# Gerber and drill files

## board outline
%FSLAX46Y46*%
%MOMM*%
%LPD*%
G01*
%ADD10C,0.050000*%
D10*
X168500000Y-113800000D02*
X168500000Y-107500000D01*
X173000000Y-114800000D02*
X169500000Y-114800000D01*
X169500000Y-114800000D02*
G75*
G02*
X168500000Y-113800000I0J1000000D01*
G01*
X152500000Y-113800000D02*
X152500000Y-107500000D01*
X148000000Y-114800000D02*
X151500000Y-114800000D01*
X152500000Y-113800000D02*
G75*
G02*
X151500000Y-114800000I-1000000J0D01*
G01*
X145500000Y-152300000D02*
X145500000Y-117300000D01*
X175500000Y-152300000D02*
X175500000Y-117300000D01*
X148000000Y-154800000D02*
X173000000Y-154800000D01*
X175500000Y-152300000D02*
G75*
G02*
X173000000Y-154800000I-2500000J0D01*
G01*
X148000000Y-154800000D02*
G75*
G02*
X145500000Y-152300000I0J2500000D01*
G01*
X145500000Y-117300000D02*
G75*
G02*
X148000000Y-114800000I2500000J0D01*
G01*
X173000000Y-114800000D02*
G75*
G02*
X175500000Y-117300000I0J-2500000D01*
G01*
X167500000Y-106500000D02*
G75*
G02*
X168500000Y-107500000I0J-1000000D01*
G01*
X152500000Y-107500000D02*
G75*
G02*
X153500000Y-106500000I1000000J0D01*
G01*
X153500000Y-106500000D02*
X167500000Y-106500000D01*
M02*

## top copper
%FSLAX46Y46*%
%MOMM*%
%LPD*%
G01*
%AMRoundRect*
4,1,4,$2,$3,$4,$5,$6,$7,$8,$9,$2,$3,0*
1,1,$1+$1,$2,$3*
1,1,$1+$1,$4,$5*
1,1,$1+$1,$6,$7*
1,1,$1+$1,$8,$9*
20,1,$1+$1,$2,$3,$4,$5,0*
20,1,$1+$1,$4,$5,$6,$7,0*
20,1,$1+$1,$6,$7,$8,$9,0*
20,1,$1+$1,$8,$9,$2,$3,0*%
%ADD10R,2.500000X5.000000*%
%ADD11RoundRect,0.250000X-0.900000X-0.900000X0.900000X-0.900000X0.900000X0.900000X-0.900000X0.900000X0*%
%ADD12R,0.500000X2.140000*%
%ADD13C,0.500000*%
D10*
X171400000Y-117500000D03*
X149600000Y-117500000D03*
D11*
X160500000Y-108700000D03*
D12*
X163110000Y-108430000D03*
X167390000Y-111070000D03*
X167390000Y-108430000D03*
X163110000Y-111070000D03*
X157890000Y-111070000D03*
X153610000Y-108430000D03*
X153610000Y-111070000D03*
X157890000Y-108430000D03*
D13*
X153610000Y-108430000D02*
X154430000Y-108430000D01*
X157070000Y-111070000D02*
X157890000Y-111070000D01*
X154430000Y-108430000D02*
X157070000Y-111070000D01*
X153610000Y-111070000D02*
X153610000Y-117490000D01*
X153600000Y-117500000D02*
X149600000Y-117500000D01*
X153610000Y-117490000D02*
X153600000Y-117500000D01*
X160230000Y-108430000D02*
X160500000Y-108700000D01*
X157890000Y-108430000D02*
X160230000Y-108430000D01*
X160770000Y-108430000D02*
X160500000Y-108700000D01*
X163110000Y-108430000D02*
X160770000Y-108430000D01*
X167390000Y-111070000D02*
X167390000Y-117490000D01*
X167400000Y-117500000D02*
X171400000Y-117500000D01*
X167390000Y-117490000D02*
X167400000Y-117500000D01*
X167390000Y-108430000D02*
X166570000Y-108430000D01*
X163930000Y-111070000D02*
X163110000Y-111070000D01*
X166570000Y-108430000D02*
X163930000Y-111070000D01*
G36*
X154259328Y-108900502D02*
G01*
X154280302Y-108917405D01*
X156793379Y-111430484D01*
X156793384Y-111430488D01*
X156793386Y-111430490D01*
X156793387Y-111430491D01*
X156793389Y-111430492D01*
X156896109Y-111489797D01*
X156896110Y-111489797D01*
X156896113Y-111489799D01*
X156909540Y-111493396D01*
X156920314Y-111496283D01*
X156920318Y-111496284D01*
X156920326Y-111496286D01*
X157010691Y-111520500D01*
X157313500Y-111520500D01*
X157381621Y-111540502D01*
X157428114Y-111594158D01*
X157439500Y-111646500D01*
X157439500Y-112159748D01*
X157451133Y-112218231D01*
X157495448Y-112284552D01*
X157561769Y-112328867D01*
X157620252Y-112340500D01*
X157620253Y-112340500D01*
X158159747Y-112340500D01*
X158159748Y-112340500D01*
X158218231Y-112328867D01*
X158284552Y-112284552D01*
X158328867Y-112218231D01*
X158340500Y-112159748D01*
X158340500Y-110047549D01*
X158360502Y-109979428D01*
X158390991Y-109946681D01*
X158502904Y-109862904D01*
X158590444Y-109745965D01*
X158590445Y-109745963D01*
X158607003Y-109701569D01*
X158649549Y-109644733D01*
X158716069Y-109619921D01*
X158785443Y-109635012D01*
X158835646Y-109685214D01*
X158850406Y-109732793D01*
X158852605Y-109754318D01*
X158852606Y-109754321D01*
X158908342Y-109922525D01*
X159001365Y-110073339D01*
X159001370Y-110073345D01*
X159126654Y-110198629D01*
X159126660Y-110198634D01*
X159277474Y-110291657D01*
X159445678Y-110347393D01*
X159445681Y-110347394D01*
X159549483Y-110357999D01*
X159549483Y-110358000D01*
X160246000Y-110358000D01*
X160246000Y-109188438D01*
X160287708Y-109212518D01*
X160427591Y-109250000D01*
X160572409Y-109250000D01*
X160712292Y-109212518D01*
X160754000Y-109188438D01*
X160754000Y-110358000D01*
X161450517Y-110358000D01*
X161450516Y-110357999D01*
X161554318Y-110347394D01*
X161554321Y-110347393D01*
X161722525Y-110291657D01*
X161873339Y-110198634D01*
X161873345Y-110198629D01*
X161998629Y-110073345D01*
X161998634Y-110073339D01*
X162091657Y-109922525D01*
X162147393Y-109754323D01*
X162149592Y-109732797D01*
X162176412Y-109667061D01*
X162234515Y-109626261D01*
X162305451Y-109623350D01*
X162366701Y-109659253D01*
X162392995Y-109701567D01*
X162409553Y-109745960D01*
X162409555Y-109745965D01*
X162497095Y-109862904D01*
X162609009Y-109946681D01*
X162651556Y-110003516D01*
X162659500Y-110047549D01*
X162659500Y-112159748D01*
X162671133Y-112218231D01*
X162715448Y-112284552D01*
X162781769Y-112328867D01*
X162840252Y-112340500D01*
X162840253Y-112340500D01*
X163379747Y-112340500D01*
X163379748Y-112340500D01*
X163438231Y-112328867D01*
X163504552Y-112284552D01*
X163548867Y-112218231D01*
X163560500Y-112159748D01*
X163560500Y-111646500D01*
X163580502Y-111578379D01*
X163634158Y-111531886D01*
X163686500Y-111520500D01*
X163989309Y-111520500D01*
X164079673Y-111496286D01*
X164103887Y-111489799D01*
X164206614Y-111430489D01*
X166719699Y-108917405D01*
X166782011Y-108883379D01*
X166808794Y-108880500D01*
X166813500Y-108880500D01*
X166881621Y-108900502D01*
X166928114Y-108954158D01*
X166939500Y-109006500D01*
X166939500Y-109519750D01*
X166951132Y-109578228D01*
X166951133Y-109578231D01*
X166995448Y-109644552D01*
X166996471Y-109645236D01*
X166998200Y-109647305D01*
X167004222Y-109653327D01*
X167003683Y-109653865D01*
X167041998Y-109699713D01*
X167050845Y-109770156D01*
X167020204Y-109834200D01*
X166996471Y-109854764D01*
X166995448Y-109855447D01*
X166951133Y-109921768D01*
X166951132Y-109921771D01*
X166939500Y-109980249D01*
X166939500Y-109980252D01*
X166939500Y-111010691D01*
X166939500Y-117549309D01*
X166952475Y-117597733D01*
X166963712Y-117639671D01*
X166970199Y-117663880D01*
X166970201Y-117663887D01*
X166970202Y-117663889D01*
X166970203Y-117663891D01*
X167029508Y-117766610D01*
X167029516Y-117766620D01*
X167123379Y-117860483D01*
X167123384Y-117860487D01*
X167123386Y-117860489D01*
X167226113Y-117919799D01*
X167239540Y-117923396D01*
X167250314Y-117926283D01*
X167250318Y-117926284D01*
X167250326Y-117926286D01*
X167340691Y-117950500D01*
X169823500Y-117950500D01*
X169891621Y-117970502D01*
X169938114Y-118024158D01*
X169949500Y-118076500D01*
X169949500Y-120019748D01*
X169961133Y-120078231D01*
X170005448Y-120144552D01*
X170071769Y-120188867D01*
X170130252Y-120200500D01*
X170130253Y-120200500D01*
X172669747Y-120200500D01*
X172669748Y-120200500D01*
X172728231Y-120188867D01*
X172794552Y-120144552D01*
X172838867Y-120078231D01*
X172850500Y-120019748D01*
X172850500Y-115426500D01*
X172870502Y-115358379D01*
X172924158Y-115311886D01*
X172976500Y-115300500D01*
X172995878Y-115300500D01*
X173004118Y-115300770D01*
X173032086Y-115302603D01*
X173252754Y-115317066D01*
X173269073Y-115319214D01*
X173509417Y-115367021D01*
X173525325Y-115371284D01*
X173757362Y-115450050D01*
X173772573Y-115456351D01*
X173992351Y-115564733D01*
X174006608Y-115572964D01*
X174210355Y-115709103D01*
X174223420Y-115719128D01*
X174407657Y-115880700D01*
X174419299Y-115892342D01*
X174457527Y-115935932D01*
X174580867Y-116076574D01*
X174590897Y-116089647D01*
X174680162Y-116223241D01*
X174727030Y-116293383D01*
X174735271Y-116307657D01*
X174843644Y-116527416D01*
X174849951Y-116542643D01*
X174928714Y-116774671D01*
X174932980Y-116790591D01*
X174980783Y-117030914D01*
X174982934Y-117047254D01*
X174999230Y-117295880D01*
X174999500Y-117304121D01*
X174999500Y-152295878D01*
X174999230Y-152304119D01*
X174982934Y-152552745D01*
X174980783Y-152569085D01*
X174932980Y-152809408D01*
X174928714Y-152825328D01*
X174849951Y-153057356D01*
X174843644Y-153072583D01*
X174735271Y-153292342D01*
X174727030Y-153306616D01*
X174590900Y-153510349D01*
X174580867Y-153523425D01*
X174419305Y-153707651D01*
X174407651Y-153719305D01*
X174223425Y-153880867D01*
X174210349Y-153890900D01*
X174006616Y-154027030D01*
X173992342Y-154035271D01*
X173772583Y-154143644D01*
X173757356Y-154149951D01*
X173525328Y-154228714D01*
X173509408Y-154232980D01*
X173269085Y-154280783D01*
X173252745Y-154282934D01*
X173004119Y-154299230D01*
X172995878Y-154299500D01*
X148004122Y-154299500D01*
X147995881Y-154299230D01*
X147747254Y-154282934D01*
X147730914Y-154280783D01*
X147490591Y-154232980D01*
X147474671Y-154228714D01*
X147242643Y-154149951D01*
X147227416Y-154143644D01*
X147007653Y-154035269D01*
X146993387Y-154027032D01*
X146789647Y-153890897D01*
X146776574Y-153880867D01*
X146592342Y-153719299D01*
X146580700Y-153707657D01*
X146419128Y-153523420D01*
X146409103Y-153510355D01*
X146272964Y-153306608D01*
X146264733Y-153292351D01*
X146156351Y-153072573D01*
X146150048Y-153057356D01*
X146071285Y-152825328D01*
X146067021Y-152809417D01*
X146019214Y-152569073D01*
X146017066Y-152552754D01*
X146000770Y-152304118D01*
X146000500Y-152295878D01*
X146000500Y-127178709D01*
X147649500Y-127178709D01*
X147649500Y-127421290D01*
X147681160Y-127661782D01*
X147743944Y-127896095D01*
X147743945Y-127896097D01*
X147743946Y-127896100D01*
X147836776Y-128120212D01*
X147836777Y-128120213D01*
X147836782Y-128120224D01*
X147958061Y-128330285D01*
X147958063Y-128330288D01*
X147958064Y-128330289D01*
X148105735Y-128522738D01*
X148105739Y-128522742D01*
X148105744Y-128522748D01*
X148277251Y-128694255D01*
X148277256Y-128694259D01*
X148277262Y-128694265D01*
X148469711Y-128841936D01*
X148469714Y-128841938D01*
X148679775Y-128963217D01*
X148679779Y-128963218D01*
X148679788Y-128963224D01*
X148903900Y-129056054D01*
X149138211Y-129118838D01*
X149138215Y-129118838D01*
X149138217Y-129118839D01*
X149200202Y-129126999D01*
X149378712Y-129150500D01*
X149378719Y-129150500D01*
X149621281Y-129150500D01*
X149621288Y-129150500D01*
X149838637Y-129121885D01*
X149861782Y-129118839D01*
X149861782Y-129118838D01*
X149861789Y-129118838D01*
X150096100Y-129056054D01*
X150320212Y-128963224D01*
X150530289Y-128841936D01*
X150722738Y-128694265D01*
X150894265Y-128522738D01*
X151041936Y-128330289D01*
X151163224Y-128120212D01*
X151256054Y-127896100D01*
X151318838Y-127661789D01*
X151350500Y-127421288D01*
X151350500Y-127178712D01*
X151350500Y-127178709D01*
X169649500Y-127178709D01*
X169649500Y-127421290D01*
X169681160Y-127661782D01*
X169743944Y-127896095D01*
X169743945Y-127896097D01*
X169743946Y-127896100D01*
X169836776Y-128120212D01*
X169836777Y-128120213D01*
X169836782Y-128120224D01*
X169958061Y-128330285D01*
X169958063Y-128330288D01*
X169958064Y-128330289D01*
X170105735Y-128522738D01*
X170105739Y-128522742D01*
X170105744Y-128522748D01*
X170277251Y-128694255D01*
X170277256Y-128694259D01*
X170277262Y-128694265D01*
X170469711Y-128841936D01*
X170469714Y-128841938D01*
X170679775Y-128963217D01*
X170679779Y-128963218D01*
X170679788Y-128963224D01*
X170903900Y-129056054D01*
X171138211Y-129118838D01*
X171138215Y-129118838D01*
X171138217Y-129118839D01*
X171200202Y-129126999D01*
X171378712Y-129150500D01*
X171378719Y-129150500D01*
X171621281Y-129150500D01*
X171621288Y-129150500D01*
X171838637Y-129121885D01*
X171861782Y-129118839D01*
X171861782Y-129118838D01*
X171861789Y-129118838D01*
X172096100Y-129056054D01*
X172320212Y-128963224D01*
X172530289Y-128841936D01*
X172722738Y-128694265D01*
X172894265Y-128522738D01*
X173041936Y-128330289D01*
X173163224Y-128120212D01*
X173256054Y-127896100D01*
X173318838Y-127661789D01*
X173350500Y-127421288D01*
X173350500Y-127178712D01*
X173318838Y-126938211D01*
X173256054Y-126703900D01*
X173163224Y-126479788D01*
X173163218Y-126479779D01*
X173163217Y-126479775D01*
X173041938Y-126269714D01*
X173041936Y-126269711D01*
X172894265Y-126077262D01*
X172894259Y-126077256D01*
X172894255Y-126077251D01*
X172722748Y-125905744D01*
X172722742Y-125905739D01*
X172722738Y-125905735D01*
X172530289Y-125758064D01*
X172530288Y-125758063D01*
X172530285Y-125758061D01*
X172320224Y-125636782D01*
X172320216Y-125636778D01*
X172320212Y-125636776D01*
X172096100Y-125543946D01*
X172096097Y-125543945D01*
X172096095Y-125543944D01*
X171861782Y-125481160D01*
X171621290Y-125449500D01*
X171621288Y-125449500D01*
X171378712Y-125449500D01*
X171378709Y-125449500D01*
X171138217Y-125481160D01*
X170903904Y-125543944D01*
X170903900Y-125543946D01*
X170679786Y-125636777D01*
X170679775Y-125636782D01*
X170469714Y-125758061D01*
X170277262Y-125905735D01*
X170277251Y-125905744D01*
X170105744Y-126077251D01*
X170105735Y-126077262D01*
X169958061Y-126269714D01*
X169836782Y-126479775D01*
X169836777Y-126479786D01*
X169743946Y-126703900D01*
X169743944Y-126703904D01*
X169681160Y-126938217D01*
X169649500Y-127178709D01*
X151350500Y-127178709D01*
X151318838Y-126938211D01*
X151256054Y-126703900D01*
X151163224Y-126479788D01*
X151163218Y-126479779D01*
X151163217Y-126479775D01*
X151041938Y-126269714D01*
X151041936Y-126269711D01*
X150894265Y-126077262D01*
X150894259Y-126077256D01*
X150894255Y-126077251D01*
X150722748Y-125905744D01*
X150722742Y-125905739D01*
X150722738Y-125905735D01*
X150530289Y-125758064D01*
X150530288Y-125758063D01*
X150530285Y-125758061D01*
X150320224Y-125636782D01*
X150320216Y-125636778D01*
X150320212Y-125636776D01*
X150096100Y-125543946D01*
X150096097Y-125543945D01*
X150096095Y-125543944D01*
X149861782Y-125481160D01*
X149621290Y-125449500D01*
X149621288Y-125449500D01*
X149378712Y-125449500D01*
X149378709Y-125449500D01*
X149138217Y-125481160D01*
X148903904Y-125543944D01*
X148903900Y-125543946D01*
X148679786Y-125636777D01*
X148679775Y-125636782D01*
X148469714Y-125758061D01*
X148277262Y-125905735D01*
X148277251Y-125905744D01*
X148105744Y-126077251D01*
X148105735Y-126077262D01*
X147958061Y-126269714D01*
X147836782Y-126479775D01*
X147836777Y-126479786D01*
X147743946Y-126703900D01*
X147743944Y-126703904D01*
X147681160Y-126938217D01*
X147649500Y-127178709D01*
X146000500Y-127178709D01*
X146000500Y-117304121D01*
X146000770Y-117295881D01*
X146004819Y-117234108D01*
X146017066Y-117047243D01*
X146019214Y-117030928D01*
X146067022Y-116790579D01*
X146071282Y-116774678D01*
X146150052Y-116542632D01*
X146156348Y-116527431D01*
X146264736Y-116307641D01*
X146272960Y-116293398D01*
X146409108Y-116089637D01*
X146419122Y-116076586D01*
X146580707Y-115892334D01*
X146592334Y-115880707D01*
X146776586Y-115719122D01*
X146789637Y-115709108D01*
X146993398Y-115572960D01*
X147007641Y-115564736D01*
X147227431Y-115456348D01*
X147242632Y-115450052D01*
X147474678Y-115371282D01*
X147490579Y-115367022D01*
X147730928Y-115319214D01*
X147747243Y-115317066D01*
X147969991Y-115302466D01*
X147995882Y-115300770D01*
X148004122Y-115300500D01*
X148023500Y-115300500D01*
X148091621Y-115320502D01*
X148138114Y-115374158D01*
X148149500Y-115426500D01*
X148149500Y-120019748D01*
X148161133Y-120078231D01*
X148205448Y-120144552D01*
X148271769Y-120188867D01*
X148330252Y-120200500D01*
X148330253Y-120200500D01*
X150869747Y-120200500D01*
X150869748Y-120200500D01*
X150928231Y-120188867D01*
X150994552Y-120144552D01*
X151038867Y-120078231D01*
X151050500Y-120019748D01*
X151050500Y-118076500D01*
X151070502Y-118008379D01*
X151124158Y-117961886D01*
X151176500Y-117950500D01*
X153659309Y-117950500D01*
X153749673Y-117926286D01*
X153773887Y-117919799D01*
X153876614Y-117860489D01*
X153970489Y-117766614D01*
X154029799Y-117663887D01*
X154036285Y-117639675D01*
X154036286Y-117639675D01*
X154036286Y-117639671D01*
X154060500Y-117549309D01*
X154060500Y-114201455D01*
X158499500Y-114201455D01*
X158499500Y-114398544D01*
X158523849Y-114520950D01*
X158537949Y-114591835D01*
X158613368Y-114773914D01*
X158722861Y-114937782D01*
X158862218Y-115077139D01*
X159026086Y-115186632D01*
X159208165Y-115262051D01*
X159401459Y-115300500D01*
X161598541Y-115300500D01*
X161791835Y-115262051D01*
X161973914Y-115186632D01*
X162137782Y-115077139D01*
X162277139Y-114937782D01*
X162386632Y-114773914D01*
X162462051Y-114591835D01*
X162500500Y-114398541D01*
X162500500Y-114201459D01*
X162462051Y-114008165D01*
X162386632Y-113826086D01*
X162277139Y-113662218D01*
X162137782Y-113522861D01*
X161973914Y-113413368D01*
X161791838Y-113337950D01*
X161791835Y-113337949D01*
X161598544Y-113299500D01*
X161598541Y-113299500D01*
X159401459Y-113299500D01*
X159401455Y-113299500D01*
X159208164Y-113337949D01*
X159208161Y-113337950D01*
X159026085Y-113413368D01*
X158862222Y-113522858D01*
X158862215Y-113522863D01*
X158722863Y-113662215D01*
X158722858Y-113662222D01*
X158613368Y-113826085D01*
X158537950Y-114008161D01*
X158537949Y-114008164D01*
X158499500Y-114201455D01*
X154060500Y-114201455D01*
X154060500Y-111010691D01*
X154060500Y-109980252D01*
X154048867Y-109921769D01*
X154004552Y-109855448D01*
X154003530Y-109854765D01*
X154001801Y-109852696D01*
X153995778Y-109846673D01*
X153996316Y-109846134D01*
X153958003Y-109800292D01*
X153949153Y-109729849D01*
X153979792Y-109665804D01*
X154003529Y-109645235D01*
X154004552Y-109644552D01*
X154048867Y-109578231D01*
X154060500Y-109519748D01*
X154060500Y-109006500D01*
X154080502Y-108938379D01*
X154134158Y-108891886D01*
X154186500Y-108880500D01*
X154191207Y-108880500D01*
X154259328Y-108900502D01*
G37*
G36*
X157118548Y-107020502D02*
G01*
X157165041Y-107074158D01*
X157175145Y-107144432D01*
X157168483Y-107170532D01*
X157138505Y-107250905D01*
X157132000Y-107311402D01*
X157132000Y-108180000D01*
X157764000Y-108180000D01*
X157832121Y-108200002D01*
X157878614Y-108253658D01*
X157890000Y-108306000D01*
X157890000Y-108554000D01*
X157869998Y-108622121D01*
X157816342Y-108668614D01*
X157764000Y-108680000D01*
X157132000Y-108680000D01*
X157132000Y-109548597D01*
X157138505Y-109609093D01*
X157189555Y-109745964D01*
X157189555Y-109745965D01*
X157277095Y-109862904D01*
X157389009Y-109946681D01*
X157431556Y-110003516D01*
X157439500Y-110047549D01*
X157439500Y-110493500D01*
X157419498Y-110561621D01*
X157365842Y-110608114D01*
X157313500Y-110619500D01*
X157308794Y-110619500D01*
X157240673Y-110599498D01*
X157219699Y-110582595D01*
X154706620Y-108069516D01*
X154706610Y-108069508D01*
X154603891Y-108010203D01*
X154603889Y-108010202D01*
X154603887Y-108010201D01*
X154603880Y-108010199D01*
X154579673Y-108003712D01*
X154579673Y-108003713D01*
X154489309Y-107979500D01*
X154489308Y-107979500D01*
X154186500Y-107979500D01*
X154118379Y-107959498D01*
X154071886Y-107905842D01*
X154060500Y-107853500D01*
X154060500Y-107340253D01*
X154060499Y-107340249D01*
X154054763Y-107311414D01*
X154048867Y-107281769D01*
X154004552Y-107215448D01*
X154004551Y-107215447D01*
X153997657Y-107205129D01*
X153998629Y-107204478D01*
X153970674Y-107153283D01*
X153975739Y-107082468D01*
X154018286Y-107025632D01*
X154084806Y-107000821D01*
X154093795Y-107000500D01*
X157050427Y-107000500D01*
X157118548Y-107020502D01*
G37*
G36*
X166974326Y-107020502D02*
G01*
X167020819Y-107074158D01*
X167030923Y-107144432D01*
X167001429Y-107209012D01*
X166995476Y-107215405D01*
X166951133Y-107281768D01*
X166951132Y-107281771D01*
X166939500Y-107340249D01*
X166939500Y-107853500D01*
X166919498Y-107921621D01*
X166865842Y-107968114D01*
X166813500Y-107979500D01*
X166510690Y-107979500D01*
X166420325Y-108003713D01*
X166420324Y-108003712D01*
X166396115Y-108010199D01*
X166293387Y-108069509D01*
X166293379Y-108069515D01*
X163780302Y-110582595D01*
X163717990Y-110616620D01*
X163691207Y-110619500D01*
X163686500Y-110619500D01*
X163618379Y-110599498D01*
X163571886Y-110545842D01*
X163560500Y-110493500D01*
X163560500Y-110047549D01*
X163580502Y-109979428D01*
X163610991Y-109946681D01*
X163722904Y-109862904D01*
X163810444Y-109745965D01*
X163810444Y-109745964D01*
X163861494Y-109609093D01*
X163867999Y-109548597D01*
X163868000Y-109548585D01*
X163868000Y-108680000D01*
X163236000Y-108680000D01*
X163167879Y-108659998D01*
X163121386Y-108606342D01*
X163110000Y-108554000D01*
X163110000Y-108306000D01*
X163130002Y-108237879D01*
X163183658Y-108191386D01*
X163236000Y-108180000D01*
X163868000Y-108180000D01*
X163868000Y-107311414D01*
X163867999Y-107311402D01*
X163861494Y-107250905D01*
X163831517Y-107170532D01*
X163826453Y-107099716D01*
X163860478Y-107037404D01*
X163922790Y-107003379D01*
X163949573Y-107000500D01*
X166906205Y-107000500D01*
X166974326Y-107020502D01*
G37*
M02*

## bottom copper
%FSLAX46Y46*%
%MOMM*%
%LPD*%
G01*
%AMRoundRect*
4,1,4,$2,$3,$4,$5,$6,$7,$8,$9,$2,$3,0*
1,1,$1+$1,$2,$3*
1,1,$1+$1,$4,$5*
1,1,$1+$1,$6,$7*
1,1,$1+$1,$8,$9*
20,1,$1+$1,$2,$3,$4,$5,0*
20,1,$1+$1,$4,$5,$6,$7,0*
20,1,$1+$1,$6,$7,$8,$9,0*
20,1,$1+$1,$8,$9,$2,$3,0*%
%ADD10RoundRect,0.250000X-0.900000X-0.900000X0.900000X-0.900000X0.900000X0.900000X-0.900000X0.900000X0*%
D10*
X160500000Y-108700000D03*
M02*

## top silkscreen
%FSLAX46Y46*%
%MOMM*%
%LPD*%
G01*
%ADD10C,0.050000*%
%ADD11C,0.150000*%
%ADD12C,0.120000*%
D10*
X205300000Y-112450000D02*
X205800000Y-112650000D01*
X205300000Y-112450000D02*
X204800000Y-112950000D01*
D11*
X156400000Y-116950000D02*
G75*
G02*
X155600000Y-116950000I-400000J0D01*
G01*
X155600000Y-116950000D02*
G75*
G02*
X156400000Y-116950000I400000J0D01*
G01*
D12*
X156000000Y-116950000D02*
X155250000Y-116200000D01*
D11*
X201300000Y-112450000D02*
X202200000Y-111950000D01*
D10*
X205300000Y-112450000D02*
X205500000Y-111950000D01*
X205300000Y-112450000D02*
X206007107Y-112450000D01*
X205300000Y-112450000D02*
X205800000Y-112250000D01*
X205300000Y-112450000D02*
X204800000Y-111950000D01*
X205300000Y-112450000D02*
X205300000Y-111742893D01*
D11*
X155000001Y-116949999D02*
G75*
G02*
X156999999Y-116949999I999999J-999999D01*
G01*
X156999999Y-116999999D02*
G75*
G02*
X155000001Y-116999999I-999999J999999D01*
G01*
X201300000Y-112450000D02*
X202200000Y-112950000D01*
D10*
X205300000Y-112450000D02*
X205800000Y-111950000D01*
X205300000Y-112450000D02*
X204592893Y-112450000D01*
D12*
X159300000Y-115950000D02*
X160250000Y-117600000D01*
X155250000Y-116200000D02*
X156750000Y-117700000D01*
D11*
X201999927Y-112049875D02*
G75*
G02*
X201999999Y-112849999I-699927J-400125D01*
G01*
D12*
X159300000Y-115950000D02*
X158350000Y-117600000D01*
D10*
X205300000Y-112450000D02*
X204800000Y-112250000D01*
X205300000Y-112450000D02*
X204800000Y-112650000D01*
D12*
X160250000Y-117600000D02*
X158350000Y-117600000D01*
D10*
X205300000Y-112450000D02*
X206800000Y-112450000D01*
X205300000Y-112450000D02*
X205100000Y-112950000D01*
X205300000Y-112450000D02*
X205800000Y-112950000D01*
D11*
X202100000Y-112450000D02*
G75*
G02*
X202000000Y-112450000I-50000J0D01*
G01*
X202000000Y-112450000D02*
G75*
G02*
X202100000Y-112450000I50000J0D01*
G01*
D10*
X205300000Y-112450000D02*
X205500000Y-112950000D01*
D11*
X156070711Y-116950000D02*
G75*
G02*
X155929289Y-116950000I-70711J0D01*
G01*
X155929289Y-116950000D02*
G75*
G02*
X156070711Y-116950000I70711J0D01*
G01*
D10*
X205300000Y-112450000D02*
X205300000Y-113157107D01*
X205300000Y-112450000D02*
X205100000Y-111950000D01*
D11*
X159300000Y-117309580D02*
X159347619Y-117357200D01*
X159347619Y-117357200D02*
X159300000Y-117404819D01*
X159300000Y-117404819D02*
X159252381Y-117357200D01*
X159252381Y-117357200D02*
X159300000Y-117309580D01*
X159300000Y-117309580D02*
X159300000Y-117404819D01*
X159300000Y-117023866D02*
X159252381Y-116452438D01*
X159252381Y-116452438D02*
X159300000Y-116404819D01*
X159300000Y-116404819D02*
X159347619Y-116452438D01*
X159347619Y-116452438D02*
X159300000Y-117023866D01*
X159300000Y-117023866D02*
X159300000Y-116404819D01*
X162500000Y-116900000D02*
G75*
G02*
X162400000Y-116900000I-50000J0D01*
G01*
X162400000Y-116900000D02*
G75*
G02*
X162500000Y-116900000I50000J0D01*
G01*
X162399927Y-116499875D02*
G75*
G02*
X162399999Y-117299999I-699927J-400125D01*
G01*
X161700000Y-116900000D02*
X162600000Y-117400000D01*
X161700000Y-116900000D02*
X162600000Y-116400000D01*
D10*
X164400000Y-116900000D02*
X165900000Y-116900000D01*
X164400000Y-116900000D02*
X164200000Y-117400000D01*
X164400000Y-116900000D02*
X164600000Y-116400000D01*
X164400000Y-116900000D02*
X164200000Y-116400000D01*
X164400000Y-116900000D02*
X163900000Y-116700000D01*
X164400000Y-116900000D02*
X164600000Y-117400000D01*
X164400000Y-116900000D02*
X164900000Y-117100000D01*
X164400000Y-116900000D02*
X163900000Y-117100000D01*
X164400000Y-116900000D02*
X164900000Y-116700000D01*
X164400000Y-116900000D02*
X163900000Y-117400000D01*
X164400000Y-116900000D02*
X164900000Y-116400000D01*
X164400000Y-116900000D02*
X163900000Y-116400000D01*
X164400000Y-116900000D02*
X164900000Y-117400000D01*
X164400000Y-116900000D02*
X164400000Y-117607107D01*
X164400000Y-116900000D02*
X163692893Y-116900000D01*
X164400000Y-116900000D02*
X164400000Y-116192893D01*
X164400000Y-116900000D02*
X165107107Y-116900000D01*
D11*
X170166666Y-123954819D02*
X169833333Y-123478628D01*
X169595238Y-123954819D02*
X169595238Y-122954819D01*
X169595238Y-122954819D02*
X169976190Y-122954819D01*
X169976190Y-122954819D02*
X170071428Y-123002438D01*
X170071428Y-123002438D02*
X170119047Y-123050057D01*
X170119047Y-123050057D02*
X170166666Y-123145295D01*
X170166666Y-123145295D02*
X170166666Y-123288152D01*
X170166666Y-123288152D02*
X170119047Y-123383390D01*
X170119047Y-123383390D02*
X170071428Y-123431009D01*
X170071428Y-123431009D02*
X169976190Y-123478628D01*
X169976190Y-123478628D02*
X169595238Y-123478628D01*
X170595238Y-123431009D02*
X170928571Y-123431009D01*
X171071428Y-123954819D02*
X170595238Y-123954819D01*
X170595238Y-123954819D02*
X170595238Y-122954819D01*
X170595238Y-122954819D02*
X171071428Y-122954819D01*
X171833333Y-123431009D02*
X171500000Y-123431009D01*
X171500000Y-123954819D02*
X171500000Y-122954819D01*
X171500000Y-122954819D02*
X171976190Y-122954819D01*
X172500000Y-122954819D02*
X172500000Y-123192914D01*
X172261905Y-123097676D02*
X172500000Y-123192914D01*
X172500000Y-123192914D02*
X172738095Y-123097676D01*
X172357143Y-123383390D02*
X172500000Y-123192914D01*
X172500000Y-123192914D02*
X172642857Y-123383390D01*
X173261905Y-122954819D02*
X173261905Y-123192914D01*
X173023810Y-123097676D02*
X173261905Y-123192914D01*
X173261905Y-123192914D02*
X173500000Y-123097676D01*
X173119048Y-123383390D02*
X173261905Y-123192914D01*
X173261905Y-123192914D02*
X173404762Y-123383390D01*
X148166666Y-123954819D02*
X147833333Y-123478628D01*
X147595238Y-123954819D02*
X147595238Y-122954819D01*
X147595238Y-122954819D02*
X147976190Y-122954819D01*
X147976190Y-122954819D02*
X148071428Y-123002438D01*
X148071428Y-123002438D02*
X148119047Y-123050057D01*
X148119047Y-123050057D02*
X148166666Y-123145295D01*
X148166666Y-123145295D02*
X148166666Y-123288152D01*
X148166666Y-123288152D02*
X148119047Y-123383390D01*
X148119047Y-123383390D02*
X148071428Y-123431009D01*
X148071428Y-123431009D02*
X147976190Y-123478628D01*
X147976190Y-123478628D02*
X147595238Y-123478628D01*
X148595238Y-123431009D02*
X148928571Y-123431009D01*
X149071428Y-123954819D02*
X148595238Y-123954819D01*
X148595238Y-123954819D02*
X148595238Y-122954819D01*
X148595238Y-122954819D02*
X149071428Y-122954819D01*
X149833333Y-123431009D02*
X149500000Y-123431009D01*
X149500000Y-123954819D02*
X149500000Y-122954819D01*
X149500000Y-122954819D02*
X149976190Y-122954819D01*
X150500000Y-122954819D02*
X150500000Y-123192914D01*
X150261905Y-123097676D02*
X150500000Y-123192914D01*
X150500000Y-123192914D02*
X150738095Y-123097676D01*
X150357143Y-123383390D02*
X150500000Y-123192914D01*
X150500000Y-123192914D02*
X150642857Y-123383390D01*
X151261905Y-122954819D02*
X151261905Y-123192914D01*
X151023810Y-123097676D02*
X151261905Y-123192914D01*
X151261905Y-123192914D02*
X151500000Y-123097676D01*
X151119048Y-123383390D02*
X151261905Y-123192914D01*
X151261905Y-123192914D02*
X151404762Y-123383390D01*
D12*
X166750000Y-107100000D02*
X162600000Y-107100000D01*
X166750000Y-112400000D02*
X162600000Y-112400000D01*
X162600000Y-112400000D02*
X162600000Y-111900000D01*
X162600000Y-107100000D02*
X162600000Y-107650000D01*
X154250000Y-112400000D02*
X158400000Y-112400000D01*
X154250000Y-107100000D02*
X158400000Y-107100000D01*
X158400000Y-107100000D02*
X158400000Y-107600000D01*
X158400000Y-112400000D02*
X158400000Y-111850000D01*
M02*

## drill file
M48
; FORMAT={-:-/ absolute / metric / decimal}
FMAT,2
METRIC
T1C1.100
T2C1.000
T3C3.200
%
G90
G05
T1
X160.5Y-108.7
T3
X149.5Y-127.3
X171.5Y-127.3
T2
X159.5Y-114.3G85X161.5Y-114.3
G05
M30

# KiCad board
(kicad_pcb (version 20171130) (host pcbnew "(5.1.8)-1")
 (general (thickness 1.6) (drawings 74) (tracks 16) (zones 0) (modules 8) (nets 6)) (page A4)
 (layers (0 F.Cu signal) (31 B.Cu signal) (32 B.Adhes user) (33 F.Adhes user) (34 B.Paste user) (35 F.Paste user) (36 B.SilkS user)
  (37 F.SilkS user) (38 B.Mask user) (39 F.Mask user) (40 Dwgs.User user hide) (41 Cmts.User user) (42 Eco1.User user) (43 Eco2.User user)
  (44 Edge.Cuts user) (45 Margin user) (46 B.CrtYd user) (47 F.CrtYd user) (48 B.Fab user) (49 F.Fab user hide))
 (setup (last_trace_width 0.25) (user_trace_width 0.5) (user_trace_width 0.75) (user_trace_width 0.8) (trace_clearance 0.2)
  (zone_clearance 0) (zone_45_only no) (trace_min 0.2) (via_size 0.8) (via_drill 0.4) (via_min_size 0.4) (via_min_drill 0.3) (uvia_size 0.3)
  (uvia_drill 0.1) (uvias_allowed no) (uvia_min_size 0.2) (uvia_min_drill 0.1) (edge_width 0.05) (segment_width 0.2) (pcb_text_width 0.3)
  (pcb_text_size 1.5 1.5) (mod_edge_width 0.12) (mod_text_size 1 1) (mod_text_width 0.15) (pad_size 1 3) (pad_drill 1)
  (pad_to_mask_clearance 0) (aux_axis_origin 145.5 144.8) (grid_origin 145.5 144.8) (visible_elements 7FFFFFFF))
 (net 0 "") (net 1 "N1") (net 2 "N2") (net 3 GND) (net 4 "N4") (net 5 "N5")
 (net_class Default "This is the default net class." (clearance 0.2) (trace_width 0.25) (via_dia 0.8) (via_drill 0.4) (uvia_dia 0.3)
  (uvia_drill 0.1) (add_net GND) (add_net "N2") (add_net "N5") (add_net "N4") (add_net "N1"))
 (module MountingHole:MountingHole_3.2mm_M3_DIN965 (layer F.Cu) (at 171.5 127.3)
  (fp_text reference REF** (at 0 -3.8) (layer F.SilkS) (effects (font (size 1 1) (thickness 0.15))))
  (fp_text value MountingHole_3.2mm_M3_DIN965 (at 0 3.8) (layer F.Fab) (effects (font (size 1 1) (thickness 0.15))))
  (pad 1 np_thru_hole circle (at 0 0) (size 3.2 3.2) (drill 3.2) (layers *.Cu *.Mask)))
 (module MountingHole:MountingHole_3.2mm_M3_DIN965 (layer F.Cu) (at 149.5 127.3)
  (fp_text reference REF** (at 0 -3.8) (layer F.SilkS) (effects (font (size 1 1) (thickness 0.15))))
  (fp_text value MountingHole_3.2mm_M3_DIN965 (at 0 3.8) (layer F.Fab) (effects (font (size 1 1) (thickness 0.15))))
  (pad 1 np_thru_hole circle (at 0 0) (size 3.2 3.2) (drill 3.2) (layers *.Cu *.Mask)))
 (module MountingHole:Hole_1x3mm (layer F.Cu) (at 160.5 114.3 90)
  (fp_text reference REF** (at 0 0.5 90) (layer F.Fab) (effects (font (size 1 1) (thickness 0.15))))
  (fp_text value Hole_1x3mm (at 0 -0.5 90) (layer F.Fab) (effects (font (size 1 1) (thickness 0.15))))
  (pad "" np_thru_hole oval (at 0 0 90) (size 1 3) (drill oval 1 3) (layers *.Cu *.Mask)))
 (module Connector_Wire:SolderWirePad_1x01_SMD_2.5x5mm (layer F.Cu) (at 171.4 117.5)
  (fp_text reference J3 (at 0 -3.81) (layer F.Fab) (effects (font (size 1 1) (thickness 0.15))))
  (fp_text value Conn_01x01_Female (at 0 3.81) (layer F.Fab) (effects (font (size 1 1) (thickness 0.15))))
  (pad 1 smd rect (at 0 0) (size 2.5 5) (layers F.Cu F.Paste F.Mask) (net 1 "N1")))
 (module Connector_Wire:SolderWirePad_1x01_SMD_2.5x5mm (layer F.Cu) (at 149.6 117.5)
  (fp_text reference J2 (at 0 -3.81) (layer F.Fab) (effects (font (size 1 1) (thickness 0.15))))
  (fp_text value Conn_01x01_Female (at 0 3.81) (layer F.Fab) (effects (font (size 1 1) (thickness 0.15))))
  (pad 1 smd rect (at 0 0) (size 2.5 5) (layers F.Cu F.Paste F.Mask) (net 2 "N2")))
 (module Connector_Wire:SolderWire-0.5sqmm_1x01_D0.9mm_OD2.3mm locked (layer F.Cu) (at 160.5 108.7)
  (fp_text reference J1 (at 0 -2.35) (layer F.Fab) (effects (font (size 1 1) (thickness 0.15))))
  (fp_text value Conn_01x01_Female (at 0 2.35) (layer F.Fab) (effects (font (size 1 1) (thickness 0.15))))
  (pad 1 thru_hole roundrect (at 0 0) (size 2.3 2.3) (drill 1.1) (layers *.Cu *.Mask) (roundrect_rratio 0.108695652173913) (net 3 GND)))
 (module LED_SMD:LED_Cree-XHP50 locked (layer F.Cu) (at 165.25 109.75)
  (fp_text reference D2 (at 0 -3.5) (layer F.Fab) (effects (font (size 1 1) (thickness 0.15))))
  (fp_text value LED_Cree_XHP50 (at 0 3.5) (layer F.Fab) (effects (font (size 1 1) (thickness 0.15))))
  (fp_line (start 1.5 -2.65) (end -2.65 -2.65) (layer F.SilkS) (width 0.12))
  (fp_line (start 1.5 2.65) (end -2.65 2.65) (layer F.SilkS) (width 0.12))
  (fp_line (start -2.65 2.65) (end -2.65 2.15) (layer F.SilkS) (width 0.12))
  (fp_line (start -2.65 -2.65) (end -2.65 -2.1) (layer F.SilkS) (width 0.12))
  (pad 2 smd rect (at -2.14 -1.32) (size 0.5 2.14) (layers F.Cu F.Paste F.Mask) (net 3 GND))
  (pad 3 smd rect (at 2.14 1.32) (size 0.5 2.14) (layers F.Cu F.Paste F.Mask) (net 1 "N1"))
  (pad 5 smd rect (at 0 0) (size 2.78 4.78) (layers F.Paste) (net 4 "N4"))
  (pad 1 smd rect (at 2.14 -1.32) (size 0.5 2.14) (layers F.Cu F.Paste F.Mask) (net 4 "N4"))
  (pad 4 smd rect (at -2.14 1.32) (size 0.5 2.14) (layers F.Cu F.Paste F.Mask) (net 4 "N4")))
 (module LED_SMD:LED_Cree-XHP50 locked (layer F.Cu) (at 155.75 109.75 180)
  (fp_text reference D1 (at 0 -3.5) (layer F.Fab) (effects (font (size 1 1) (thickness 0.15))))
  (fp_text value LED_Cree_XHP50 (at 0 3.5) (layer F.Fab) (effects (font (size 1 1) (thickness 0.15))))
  (fp_line (start 1.5 -2.65) (end -2.65 -2.65) (layer F.SilkS) (width 0.12))
  (fp_line (start 1.5 2.65) (end -2.65 2.65) (layer F.SilkS) (width 0.12))
  (fp_line (start -2.65 2.65) (end -2.65 2.15) (layer F.SilkS) (width 0.12))
  (fp_line (start -2.65 -2.65) (end -2.65 -2.1) (layer F.SilkS) (width 0.12))
  (pad 2 smd rect (at -2.14 -1.32 180) (size 0.5 2.14) (layers F.Cu F.Paste F.Mask) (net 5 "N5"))
  (pad 3 smd rect (at 2.14 1.32 180) (size 0.5 2.14) (layers F.Cu F.Paste F.Mask) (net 5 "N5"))
  (pad 5 smd rect (at 0 0 180) (size 2.78 4.78) (layers F.Paste) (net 5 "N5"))
  (pad 1 smd rect (at 2.14 -1.32 180) (size 0.5 2.14) (layers F.Cu F.Paste F.Mask) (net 2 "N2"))
  (pad 4 smd rect (at -2.14 1.32 180) (size 0.5 2.14) (layers F.Cu F.Paste F.Mask) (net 3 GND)))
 (gr_line (start 205.3 112.45) (end 205.8 112.65) (layer F.SilkS) (width 0.05))
 (gr_line (start 205.3 112.45) (end 204.8 112.95) (layer F.SilkS) (width 0.05))
 (gr_circle (center 156 116.95) (end 156.4 116.95) (layer F.SilkS) (width 0.15))
 (gr_line (start 156 116.95) (end 155.25 116.2) (layer F.SilkS) (width 0.12))
 (gr_line (start 201.3 112.45) (end 202.2 111.95) (layer F.SilkS) (width 0.15))
 (gr_line (start 205.3 112.45) (end 205.5 111.95) (layer F.SilkS) (width 0.05))
 (gr_line (start 205.3 112.45) (end 206.007107 112.45) (layer F.SilkS) (width 0.05))
 (gr_line (start 205.3 112.45) (end 205.8 112.25) (layer F.SilkS) (width 0.05))
 (gr_line (start 205.3 112.45) (end 204.8 111.95) (layer F.SilkS) (width 0.05))
 (gr_line (start 205.3 112.45) (end 205.3 111.742893) (layer F.SilkS) (width 0.05))
 (gr_arc (start 156 117.949998) (end 156.999999 116.949999) (angle -90) (layer F.SilkS) (width 0.15))
 (gr_arc (start 156 116) (end 155.000001 116.999999) (angle -90) (layer F.SilkS) (width 0.15))
 (gr_line (start 201.3 112.45) (end 202.2 112.95) (layer F.SilkS) (width 0.15))
 (gr_line (start 205.3 112.45) (end 205.8 111.95) (layer F.SilkS) (width 0.05))
 (gr_line (start 205.3 112.45) (end 204.592893 112.45) (layer F.SilkS) (width 0.05))
 (gr_line (start 159.3 115.95) (end 160.25 117.6) (layer F.SilkS) (width 0.12))
 (gr_line (start 155.25 116.2) (end 156.75 117.7) (layer F.SilkS) (width 0.12))
 (gr_arc (start 201.3 112.45) (end 201.999999 112.849999) (angle -59.5) (layer F.SilkS) (width 0.15))
 (gr_line (start 159.3 115.95) (end 158.35 117.6) (layer F.SilkS) (width 0.12))
 (gr_line (start 205.3 112.45) (end 204.8 112.25) (layer F.SilkS) (width 0.05))
 (gr_line (start 205.3 112.45) (end 204.8 112.65) (layer F.SilkS) (width 0.05))
 (gr_line (start 160.25 117.6) (end 158.35 117.6) (layer F.SilkS) (width 0.12))
 (gr_line (start 205.3 112.45) (end 206.8 112.45) (layer F.SilkS) (width 0.05))
 (gr_line (start 205.3 112.45) (end 205.1 112.95) (layer F.SilkS) (width 0.05))
 (gr_line (start 205.3 112.45) (end 205.8 112.95) (layer F.SilkS) (width 0.05))
 (gr_circle (center 202.05 112.45) (end 202.1 112.45) (layer F.SilkS) (width 0.15))
 (gr_line (start 205.3 112.45) (end 205.5 112.95) (layer F.SilkS) (width 0.05))
 (gr_circle (center 156 116.95) (end 156.070711 116.95) (layer F.SilkS) (width 0.15))
 (gr_line (start 205.3 112.45) (end 205.3 113.157107) (layer F.SilkS) (width 0.05))
 (gr_line (start 205.3 112.45) (end 205.1 111.95) (layer F.SilkS) (width 0.05))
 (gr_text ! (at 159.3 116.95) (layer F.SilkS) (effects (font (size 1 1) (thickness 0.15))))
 (gr_line (start 168.5 113.8) (end 168.5 107.5) (layer Edge.Cuts) (width 0.05))
 (gr_line (start 173 114.8) (end 169.5 114.8) (layer Edge.Cuts) (width 0.05))
 (gr_arc (start 169.5 113.8) (end 168.5 113.8) (angle -90) (layer Edge.Cuts) (width 0.05))
 (gr_line (start 152.5 113.8) (end 152.5 107.5) (layer Edge.Cuts) (width 0.05))
 (gr_line (start 148 114.8) (end 151.5 114.8) (layer Edge.Cuts) (width 0.05))
 (gr_arc (start 151.5 113.8) (end 151.5 114.8) (angle -90) (layer Edge.Cuts) (width 0.05))
 (gr_line (start 145.5 152.3) (end 145.5 117.3) (layer Edge.Cuts) (width 0.05))
 (gr_line (start 175.5 152.3) (end 175.5 117.3) (layer Edge.Cuts) (width 0.05))
 (gr_line (start 148 154.8) (end 173 154.8) (layer Edge.Cuts) (width 0.05))
 (gr_arc (start 173 152.3) (end 173 154.8) (angle -90) (layer Edge.Cuts) (width 0.05))
 (gr_arc (start 148 152.3) (end 145.5 152.3) (angle -90) (layer Edge.Cuts) (width 0.05))
 (gr_arc (start 148 117.3) (end 148 114.8) (angle -90) (layer Edge.Cuts) (width 0.05))
 (gr_arc (start 173 117.3) (end 175.5 117.3) (angle -90) (layer Edge.Cuts) (width 0.05))
 (gr_arc (start 167.5 107.5) (end 168.5 107.5) (angle -90) (layer Edge.Cuts) (width 0.05))
 (gr_arc (start 153.5 107.5) (end 153.5 106.5) (angle -90) (layer Edge.Cuts) (width 0.05))
 (gr_line (start 153.5 106.5) (end 167.5 106.5) (layer Edge.Cuts) (width 0.05))
 (gr_circle (center 162.45 116.9) (end 162.5 116.9) (layer F.SilkS) (width 0.15))
 (gr_arc (start 161.7 116.9) (end 162.399999 117.299999) (angle -59.5) (layer F.SilkS) (width 0.15))
 (gr_line (start 161.7 116.9) (end 162.6 117.4) (layer F.SilkS) (width 0.15))
 (gr_line (start 161.7 116.9) (end 162.6 116.4) (layer F.SilkS) (width 0.15))
 (gr_line (start 164.4 116.9) (end 165.9 116.9) (layer F.SilkS) (width 0.05))
 (gr_line (start 164.4 116.9) (end 164.2 117.4) (layer F.SilkS) (width 0.05))
 (gr_line (start 164.4 116.9) (end 164.6 116.4) (layer F.SilkS) (width 0.05))
 (gr_line (start 164.4 116.9) (end 164.2 116.4) (layer F.SilkS) (width 0.05))
 (gr_line (start 164.4 116.9) (end 163.9 116.7) (layer F.SilkS) (width 0.05))
 (gr_line (start 164.4 116.9) (end 164.6 117.4) (layer F.SilkS) (width 0.05))
 (gr_line (start 164.4 116.9) (end 164.9 117.1) (layer F.SilkS) (width 0.05))
 (gr_line (start 164.4 116.9) (end 163.9 117.1) (layer F.SilkS) (width 0.05))
 (gr_line (start 164.4 116.9) (end 164.9 116.7) (layer F.SilkS) (width 0.05))
 (gr_line (start 164.4 116.9) (end 163.9 117.4) (layer F.SilkS) (width 0.05))
 (gr_line (start 164.4 116.9) (end 164.9 116.4) (layer F.SilkS) (width 0.05))
 (gr_line (start 164.4 116.9) (end 163.9 116.4) (layer F.SilkS) (width 0.05))
 (gr_line (start 164.4 116.9) (end 164.9 117.4) (layer F.SilkS) (width 0.05))
 (gr_line (start 164.4 116.9) (end 164.4 117.607107) (layer F.SilkS) (width 0.05))
 (gr_line (start 164.4 116.9) (end 163.692893 116.9) (layer F.SilkS) (width 0.05))
 (gr_line (start 164.4 116.9) (end 164.4 116.192893) (layer F.SilkS) (width 0.05))
 (gr_line (start 164.4 116.9) (end 165.107107 116.9) (layer F.SilkS) (width 0.05))
 (segment (start 153.61 108.43) (end 154.43 108.43) (width 0.5) (layer F.Cu) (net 5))
 (segment (start 157.07 111.07) (end 157.89 111.07) (width 0.5) (layer F.Cu) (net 5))
 (segment (start 154.43 108.43) (end 157.07 111.07) (width 0.5) (layer F.Cu) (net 5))
 (segment (start 153.61 111.07) (end 153.61 117.49) (width 0.5) (layer F.Cu) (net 2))
 (segment (start 153.6 117.5) (end 149.6 117.5) (width 0.5) (layer F.Cu) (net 2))
 (segment (start 153.61 117.49) (end 153.6 117.5) (width 0.5) (layer F.Cu) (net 2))
 (segment (start 160.23 108.43) (end 160.5 108.7) (width 0.5) (layer F.Cu) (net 3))
 (segment (start 157.89 108.43) (end 160.23 108.43) (width 0.5) (layer F.Cu) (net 3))
 (segment (start 160.77 108.43) (end 160.5 108.7) (width 0.5) (layer F.Cu) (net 3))
 (segment (start 163.11 108.43) (end 160.77 108.43) (width 0.5) (layer F.Cu) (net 3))
 (segment (start 167.39 111.07) (end 167.39 117.49) (width 0.5) (layer F.Cu) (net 1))
 (segment (start 167.4 117.5) (end 171.4 117.5) (width 0.5) (layer F.Cu) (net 1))
 (segment (start 167.39 117.49) (end 167.4 117.5) (width 0.5) (layer F.Cu) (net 1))
 (segment (start 167.39 108.43) (end 166.57 108.43) (width 0.5) (layer F.Cu) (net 4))
 (segment (start 163.93 111.07) (end 163.11 111.07) (width 0.5) (layer F.Cu) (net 4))
 (segment (start 166.57 108.43) (end 163.93 111.07) (width 0.5) (layer F.Cu) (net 4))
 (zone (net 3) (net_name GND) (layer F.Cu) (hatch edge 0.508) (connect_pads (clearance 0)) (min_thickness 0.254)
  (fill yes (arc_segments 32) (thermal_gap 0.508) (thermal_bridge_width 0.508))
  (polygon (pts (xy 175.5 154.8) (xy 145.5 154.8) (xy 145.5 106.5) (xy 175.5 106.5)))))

